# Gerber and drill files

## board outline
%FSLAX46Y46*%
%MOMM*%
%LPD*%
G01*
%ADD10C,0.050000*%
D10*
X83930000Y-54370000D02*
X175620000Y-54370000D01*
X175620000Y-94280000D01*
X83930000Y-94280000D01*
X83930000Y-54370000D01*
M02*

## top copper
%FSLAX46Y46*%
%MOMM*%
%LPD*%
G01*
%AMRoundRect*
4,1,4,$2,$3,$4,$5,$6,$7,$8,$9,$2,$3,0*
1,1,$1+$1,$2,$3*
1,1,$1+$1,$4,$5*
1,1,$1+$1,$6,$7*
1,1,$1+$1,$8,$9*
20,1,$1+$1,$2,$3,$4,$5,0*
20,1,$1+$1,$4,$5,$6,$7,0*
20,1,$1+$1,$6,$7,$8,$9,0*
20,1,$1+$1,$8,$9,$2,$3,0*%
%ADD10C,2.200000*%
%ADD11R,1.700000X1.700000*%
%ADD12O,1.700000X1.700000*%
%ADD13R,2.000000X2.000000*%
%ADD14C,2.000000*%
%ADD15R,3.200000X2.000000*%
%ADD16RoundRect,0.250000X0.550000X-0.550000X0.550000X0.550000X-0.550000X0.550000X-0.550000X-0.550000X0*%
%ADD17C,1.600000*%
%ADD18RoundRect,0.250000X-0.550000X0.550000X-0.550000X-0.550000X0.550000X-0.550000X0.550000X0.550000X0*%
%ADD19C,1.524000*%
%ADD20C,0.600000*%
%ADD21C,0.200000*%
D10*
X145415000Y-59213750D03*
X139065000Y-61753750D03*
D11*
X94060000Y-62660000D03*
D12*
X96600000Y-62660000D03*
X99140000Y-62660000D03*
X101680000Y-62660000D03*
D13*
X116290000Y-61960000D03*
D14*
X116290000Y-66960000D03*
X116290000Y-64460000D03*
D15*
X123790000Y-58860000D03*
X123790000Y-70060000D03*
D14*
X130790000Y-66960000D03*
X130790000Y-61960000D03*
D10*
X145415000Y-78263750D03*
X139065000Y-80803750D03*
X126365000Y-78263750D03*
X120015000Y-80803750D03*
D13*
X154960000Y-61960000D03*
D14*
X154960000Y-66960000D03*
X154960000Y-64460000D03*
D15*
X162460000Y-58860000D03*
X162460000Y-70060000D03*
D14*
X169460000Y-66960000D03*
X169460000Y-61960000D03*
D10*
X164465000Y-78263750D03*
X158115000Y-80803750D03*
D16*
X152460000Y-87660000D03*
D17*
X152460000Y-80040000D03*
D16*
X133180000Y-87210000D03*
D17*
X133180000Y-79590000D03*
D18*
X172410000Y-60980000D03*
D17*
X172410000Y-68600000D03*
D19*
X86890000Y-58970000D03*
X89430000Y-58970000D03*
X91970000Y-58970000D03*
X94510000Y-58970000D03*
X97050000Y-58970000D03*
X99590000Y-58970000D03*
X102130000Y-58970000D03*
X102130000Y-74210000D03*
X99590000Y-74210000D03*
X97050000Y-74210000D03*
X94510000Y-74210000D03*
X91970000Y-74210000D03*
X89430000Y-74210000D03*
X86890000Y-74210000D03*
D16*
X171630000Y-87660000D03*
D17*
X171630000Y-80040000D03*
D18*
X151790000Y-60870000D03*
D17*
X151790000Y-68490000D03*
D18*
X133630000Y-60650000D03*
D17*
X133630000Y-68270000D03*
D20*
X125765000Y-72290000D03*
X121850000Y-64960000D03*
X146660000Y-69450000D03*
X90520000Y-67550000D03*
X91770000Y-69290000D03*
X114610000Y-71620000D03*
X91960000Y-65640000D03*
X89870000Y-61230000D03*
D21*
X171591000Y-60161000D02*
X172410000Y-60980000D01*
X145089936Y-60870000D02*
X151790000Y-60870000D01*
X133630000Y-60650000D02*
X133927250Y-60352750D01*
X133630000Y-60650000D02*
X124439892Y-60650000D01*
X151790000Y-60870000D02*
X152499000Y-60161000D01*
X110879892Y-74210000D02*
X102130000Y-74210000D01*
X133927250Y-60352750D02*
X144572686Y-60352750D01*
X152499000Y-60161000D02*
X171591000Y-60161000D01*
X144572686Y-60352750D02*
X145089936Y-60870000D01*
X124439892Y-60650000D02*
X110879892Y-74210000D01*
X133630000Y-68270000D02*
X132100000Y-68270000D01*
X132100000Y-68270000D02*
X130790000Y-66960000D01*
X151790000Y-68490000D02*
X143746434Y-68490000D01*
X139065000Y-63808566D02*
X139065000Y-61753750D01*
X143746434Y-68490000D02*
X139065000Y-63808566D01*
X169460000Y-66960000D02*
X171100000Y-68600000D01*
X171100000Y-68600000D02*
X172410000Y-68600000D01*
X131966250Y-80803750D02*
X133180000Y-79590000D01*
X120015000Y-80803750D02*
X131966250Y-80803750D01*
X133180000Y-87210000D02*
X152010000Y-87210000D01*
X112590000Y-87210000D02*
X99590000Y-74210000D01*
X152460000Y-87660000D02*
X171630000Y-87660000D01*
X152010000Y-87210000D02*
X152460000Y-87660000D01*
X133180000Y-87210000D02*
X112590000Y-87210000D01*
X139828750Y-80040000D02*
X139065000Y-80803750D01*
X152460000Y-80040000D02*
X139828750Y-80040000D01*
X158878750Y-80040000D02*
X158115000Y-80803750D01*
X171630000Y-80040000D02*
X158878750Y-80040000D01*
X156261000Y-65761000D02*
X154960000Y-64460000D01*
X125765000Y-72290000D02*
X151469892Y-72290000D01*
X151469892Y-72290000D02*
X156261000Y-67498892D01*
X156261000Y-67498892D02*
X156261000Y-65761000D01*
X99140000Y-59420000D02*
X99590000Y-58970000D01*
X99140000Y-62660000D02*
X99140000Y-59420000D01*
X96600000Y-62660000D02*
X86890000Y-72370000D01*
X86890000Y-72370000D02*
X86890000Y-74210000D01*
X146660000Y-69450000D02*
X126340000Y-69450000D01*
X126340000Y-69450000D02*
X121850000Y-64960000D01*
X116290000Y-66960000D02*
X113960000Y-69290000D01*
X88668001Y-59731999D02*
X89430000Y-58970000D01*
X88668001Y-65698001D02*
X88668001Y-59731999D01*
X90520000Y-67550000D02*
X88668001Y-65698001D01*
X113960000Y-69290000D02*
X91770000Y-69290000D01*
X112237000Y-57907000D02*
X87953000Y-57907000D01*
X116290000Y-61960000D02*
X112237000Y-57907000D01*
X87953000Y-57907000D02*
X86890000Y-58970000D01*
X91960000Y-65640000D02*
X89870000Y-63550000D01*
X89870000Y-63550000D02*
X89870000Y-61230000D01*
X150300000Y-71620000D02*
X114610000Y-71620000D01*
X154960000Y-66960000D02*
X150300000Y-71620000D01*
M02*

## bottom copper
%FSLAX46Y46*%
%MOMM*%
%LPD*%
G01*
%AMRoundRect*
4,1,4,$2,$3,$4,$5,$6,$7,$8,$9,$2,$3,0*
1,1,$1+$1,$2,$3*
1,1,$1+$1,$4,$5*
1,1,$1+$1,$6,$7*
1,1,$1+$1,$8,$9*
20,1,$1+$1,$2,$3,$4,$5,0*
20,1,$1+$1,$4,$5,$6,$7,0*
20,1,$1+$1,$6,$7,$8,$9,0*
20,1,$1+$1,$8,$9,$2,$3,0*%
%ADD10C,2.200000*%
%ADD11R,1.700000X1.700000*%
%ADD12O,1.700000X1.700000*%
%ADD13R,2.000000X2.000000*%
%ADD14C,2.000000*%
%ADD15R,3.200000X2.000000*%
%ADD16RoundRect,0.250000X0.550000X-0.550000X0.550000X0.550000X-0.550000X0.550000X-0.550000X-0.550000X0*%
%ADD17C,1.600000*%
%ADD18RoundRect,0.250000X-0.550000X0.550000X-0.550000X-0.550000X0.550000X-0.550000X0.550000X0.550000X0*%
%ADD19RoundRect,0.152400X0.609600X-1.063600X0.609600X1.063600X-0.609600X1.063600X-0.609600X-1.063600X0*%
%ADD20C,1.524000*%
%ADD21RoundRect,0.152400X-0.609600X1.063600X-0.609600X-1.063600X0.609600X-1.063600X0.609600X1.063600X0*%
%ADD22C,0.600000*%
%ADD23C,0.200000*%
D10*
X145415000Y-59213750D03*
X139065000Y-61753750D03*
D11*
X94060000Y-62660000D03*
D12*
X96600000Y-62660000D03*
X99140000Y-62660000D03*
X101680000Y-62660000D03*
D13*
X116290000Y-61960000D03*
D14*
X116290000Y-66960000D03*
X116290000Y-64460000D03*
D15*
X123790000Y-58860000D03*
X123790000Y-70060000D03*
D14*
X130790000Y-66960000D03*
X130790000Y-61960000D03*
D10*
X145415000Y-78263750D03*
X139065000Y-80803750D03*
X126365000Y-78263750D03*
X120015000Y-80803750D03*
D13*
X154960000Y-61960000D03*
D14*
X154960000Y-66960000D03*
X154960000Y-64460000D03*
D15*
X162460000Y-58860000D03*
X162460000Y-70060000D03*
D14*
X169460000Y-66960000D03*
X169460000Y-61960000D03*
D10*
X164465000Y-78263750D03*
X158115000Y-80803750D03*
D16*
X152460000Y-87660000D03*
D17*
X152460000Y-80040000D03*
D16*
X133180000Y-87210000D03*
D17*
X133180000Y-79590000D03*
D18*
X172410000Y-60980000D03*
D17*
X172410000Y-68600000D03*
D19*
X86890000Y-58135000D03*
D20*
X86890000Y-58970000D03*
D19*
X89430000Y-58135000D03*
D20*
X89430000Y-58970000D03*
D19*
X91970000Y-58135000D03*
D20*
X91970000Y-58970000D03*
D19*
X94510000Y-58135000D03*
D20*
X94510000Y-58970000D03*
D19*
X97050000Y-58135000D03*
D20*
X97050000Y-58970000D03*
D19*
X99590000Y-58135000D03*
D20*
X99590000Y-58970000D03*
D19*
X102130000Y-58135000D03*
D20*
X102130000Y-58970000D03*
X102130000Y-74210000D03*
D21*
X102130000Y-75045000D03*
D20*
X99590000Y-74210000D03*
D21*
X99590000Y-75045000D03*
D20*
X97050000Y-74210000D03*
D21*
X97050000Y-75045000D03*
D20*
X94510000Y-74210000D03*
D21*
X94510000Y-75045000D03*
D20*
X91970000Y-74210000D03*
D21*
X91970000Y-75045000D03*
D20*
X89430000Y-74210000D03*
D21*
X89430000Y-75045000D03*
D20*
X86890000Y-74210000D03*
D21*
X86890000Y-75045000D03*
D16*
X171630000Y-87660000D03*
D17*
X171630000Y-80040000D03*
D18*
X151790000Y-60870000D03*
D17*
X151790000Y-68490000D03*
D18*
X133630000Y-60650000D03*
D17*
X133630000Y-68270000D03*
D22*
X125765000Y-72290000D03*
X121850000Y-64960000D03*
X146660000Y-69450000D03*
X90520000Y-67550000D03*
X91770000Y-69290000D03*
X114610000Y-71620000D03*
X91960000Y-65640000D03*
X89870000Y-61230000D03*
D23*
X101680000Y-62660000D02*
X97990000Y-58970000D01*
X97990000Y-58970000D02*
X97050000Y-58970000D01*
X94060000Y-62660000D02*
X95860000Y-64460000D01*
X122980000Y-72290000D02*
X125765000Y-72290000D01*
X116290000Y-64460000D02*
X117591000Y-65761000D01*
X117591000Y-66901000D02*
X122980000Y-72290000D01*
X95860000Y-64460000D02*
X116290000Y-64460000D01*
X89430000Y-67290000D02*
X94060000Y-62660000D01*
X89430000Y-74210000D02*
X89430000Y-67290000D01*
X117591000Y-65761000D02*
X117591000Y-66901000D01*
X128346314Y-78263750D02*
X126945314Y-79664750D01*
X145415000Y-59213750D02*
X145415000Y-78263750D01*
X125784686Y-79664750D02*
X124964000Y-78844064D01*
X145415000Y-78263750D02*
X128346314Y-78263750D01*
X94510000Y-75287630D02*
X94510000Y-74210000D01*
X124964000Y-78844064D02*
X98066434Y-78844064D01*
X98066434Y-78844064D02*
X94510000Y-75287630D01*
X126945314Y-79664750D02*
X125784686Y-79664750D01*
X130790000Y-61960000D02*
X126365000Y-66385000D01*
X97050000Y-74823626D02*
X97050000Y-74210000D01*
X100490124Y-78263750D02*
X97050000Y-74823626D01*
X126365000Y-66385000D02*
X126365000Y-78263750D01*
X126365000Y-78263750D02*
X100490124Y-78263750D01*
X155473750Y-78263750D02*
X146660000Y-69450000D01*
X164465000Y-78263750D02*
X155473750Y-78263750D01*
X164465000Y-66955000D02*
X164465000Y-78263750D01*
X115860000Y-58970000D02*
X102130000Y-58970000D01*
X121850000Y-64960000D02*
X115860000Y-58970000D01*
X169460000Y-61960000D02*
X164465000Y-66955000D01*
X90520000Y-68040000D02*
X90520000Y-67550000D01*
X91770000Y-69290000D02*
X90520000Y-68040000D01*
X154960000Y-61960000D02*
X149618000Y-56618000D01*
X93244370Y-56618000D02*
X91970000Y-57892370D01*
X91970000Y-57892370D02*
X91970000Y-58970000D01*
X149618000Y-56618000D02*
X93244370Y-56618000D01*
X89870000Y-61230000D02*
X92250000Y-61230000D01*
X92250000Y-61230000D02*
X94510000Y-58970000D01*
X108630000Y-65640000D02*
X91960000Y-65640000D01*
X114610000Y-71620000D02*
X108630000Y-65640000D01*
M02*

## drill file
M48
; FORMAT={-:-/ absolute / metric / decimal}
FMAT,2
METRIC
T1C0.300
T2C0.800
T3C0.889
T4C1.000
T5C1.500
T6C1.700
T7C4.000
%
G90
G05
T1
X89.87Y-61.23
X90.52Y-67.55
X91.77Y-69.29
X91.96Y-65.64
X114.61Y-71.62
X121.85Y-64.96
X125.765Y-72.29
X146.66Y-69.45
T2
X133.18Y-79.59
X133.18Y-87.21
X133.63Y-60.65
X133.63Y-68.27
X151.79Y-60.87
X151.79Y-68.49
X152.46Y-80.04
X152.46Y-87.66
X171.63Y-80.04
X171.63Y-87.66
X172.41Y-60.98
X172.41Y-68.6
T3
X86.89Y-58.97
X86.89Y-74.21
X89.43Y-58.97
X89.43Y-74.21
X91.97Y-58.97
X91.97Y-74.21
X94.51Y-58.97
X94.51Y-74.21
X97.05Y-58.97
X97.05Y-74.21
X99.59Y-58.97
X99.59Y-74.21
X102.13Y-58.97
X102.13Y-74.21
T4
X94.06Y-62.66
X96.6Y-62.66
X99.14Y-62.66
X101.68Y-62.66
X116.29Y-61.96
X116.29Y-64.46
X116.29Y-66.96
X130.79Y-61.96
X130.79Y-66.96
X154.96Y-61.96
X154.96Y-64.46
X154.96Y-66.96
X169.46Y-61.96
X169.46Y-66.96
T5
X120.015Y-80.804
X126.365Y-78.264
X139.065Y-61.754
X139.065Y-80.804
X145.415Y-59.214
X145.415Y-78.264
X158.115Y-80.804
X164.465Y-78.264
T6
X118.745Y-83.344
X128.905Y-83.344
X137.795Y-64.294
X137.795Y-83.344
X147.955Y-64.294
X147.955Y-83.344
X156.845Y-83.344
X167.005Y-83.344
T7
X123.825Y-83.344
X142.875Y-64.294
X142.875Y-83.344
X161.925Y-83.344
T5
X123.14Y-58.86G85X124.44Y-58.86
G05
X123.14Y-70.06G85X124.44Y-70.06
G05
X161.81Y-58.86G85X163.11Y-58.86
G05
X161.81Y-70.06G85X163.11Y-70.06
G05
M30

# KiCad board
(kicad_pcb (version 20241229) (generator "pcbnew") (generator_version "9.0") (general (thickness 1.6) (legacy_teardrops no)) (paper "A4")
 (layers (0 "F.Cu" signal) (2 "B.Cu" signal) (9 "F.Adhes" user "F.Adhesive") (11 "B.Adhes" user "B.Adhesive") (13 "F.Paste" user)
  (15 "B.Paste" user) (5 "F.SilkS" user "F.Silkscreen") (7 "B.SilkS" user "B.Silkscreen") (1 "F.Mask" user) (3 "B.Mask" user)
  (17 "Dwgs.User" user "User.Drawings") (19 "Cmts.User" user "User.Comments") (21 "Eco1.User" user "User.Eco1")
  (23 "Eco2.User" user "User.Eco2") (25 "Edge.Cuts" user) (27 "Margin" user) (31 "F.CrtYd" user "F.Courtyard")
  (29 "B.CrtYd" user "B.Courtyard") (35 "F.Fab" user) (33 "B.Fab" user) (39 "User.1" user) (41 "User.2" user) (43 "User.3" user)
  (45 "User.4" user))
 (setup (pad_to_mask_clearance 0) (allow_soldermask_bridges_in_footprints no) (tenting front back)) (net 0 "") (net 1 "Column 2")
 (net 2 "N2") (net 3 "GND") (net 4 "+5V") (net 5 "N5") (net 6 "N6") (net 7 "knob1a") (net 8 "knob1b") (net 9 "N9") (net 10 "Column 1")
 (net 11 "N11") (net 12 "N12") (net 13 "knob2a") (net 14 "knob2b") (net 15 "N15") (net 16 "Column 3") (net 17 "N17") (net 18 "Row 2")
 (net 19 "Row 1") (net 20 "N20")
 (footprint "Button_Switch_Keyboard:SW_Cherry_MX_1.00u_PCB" (layer "F.Cu") (at 145.415 59.21375)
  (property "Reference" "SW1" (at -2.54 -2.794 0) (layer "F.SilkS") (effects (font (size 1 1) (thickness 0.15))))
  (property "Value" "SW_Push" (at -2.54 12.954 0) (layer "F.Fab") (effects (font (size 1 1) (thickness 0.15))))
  (pad "" np_thru_hole circle (at -7.62 5.08) (size 1.7 1.7) (drill 1.7) (layers "*.Cu" "*.Mask"))
  (pad "" np_thru_hole circle (at -2.54 5.08) (size 4 4) (drill 4) (layers "*.Cu" "*.Mask"))
  (pad "" np_thru_hole circle (at 2.54 5.08) (size 1.7 1.7) (drill 1.7) (layers "*.Cu" "*.Mask"))
  (pad "1" thru_hole circle (at 0 0) (size 2.2 2.2) (drill 1.5) (layers "*.Cu" "*.Mask") (remove_unused_layers no) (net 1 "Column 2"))
  (pad "2" thru_hole circle (at -6.35 2.54) (size 2.2 2.2) (drill 1.5) (layers "*.Cu" "*.Mask") (remove_unused_layers no) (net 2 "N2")))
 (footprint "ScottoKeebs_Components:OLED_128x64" (layer "F.Cu") (at 97.87 62.66)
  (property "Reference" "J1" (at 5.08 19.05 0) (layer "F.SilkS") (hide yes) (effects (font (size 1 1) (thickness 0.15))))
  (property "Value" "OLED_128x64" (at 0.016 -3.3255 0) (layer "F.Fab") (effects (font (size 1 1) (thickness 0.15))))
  (pad "1" thru_hole rect (at -3.81 0 90) (size 1.7 1.7) (drill 1) (layers "*.Cu" "*.Mask") (remove_unused_layers no) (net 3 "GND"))
  (pad "2" thru_hole oval (at -1.27 0 90) (size 1.7 1.7) (drill 1) (layers "*.Cu" "*.Mask") (remove_unused_layers no) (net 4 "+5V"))
  (pad "3" thru_hole oval (at 1.27 0 90) (size 1.7 1.7) (drill 1) (layers "*.Cu" "*.Mask") (remove_unused_layers no) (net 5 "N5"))
  (pad "4" thru_hole oval (at 3.81 0 90) (size 1.7 1.7) (drill 1) (layers "*.Cu" "*.Mask") (remove_unused_layers no) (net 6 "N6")))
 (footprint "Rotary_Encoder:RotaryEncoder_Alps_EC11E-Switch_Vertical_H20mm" (layer "F.Cu") (at 116.29 61.96)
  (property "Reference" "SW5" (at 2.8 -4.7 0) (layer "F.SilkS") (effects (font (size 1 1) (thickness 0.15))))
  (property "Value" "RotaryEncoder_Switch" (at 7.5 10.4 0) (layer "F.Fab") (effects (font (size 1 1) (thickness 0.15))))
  (pad "A" thru_hole rect (at 0 0) (size 2 2) (drill 1) (layers "*.Cu" "*.Mask") (remove_unused_layers no) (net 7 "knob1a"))
  (pad "B" thru_hole circle (at 0 5) (size 2 2) (drill 1) (layers "*.Cu" "*.Mask") (remove_unused_layers no) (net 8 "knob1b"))
  (pad "C" thru_hole circle (at 0 2.5) (size 2 2) (drill 1) (layers "*.Cu" "*.Mask") (remove_unused_layers no) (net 3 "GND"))
  (pad "MP" thru_hole rect (at 7.5 -3.1) (size 3.2 2) (drill oval 2.8 1.5) (layers "*.Cu" "*.Mask") (remove_unused_layers no))
  (pad "MP" thru_hole rect (at 7.5 8.1) (size 3.2 2) (drill oval 2.8 1.5) (layers "*.Cu" "*.Mask") (remove_unused_layers no))
  (pad "S1" thru_hole circle (at 14.5 5) (size 2 2) (drill 1) (layers "*.Cu" "*.Mask") (remove_unused_layers no) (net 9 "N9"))
  (pad "S2" thru_hole circle (at 14.5 0) (size 2 2) (drill 1) (layers "*.Cu" "*.Mask") (remove_unused_layers no) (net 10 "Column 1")))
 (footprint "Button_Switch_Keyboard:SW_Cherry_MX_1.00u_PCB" (layer "F.Cu") (at 145.415 78.26375)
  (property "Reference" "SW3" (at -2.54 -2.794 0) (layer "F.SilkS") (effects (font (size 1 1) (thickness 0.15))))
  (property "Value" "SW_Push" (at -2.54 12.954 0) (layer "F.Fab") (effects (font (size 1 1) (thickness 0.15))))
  (pad "" np_thru_hole circle (at -7.62 5.08) (size 1.7 1.7) (drill 1.7) (layers "*.Cu" "*.Mask"))
  (pad "" np_thru_hole circle (at -2.54 5.08) (size 4 4) (drill 4) (layers "*.Cu" "*.Mask"))
  (pad "" np_thru_hole circle (at 2.54 5.08) (size 1.7 1.7) (drill 1.7) (layers "*.Cu" "*.Mask"))
  (pad "1" thru_hole circle (at 0 0) (size 2.2 2.2) (drill 1.5) (layers "*.Cu" "*.Mask") (remove_unused_layers no) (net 1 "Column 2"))
  (pad "2" thru_hole circle (at -6.35 2.54) (size 2.2 2.2) (drill 1.5) (layers "*.Cu" "*.Mask") (remove_unused_layers no) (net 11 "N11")))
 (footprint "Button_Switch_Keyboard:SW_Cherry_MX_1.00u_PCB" (layer "F.Cu") (at 126.365 78.26375)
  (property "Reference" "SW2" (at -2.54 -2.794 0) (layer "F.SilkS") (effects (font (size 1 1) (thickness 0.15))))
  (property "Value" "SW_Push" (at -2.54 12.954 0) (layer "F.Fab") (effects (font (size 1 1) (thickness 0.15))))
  (pad "" np_thru_hole circle (at -7.62 5.08) (size 1.7 1.7) (drill 1.7) (layers "*.Cu" "*.Mask"))
  (pad "" np_thru_hole circle (at -2.54 5.08) (size 4 4) (drill 4) (layers "*.Cu" "*.Mask"))
  (pad "" np_thru_hole circle (at 2.54 5.08) (size 1.7 1.7) (drill 1.7) (layers "*.Cu" "*.Mask"))
  (pad "1" thru_hole circle (at 0 0) (size 2.2 2.2) (drill 1.5) (layers "*.Cu" "*.Mask") (remove_unused_layers no) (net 10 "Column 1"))
  (pad "2" thru_hole circle (at -6.35 2.54) (size 2.2 2.2) (drill 1.5) (layers "*.Cu" "*.Mask") (remove_unused_layers no) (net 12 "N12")))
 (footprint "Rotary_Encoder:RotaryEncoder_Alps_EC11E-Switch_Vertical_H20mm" (layer "F.Cu") (at 154.96 61.96)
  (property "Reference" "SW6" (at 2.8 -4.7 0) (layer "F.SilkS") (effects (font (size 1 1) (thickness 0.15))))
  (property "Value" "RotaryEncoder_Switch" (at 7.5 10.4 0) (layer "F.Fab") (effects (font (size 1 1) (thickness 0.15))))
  (pad "A" thru_hole rect (at 0 0) (size 2 2) (drill 1) (layers "*.Cu" "*.Mask") (remove_unused_layers no) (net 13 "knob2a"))
  (pad "B" thru_hole circle (at 0 5) (size 2 2) (drill 1) (layers "*.Cu" "*.Mask") (remove_unused_layers no) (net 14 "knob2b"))
  (pad "C" thru_hole circle (at 0 2.5) (size 2 2) (drill 1) (layers "*.Cu" "*.Mask") (remove_unused_layers no) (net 3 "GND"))
  (pad "MP" thru_hole rect (at 7.5 -3.1) (size 3.2 2) (drill oval 2.8 1.5) (layers "*.Cu" "*.Mask") (remove_unused_layers no))
  (pad "MP" thru_hole rect (at 7.5 8.1) (size 3.2 2) (drill oval 2.8 1.5) (layers "*.Cu" "*.Mask") (remove_unused_layers no))
  (pad "S1" thru_hole circle (at 14.5 5) (size 2 2) (drill 1) (layers "*.Cu" "*.Mask") (remove_unused_layers no) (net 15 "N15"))
  (pad "S2" thru_hole circle (at 14.5 0) (size 2 2) (drill 1) (layers "*.Cu" "*.Mask") (remove_unused_layers no) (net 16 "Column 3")))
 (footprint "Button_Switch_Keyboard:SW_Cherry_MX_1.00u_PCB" (layer "F.Cu") (at 164.465 78.26375)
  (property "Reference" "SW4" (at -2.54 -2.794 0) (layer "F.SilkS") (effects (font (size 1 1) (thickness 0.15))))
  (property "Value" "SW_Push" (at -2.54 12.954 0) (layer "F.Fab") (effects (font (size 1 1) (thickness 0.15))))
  (pad "" np_thru_hole circle (at -7.62 5.08) (size 1.7 1.7) (drill 1.7) (layers "*.Cu" "*.Mask"))
  (pad "" np_thru_hole circle (at -2.54 5.08) (size 4 4) (drill 4) (layers "*.Cu" "*.Mask"))
  (pad "" np_thru_hole circle (at 2.54 5.08) (size 1.7 1.7) (drill 1.7) (layers "*.Cu" "*.Mask"))
  (pad "1" thru_hole circle (at 0 0) (size 2.2 2.2) (drill 1.5) (layers "*.Cu" "*.Mask") (remove_unused_layers no) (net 16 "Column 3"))
  (pad "2" thru_hole circle (at -6.35 2.54) (size 2.2 2.2) (drill 1.5) (layers "*.Cu" "*.Mask") (remove_unused_layers no) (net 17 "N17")))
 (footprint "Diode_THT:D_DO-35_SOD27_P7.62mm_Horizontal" (layer "B.Cu") (at 152.46 87.66 90)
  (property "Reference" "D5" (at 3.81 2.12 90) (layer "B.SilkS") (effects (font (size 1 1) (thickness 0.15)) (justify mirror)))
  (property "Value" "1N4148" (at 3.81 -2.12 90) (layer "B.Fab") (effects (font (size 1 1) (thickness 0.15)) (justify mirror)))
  (pad "1" thru_hole roundrect (at 0 0 90) (size 1.6 1.6) (drill 0.8) (layers "*.Cu" "*.Mask") (remove_unused_layers no)
   (roundrect_rratio 0.15625) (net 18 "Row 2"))
  (pad "2" thru_hole circle (at 7.62 0 90) (size 1.6 1.6) (drill 0.8) (layers "*.Cu" "*.Mask") (remove_unused_layers no) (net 11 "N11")))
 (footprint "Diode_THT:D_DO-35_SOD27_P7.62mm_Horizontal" (layer "B.Cu") (at 133.18 87.21 90)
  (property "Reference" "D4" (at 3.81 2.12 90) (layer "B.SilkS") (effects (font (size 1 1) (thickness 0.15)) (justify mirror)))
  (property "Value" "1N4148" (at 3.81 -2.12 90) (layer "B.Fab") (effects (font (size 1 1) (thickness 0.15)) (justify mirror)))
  (pad "1" thru_hole roundrect (at 0 0 90) (size 1.6 1.6) (drill 0.8) (layers "*.Cu" "*.Mask") (remove_unused_layers no)
   (roundrect_rratio 0.15625) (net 18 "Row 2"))
  (pad "2" thru_hole circle (at 7.62 0 90) (size 1.6 1.6) (drill 0.8) (layers "*.Cu" "*.Mask") (remove_unused_layers no) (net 12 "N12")))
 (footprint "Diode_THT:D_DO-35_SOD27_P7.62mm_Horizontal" (layer "B.Cu") (at 172.41 60.98 -90)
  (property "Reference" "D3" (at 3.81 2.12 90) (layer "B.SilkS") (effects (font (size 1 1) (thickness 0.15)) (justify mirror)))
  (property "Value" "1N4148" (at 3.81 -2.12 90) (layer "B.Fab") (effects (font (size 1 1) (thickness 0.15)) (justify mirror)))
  (pad "1" thru_hole roundrect (at 0 0 270) (size 1.6 1.6) (drill 0.8) (layers "*.Cu" "*.Mask") (remove_unused_layers no)
   (roundrect_rratio 0.15625) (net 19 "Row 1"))
  (pad "2" thru_hole circle (at 7.62 0 270) (size 1.6 1.6) (drill 0.8) (layers "*.Cu" "*.Mask") (remove_unused_layers no) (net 15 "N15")))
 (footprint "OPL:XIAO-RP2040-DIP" (layer "B.Cu") (at 94.51 66.59 -90)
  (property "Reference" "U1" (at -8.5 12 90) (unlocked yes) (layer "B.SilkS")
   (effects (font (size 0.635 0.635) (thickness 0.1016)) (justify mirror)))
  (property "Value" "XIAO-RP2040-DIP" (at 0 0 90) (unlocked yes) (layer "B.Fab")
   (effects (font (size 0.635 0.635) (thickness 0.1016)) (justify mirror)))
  (pad "1" smd roundrect (at -8.455 7.62 90) (size 2.432 1.524) (layers "B.Cu" "B.Mask") (roundrect_rratio 0.1) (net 7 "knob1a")
   (thermal_bridge_angle 45))
  (pad "1" thru_hole circle (at -7.62 7.62 90) (size 1.524 1.524) (drill 0.889) (layers "*.Cu" "*.Mask") (remove_unused_layers no)
   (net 7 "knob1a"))
  (pad "2" smd roundrect (at -8.455 5.08 90) (size 2.432 1.524) (layers "B.Cu" "B.Mask") (roundrect_rratio 0.1) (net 8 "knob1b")
   (thermal_bridge_angle 45))
  (pad "2" thru_hole circle (at -7.62 5.08 90) (size 1.524 1.524) (drill 0.889) (layers "*.Cu" "*.Mask") (remove_unused_layers no)
   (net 8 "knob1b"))
  (pad "3" smd roundrect (at -8.455 2.54 90) (size 2.432 1.524) (layers "B.Cu" "B.Mask") (roundrect_rratio 0.1) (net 13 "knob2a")
   (thermal_bridge_angle 45))
  (pad "3" thru_hole circle (at -7.62 2.54 90) (size 1.524 1.524) (drill 0.889) (layers "*.Cu" "*.Mask") (remove_unused_layers no)
   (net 13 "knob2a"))
  (pad "4" smd roundrect (at -8.455 0 90) (size 2.432 1.524) (layers "B.Cu" "B.Mask") (roundrect_rratio 0.1) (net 14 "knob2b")
   (thermal_bridge_angle 45))
  (pad "4" thru_hole circle (at -7.62 0 90) (size 1.524 1.524) (drill 0.889) (layers "*.Cu" "*.Mask") (remove_unused_layers no)
   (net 14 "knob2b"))
  (pad "5" smd roundrect (at -8.455 -2.54 90) (size 2.432 1.524) (layers "B.Cu" "B.Mask") (roundrect_rratio 0.1) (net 6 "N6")
   (thermal_bridge_angle 45))
  (pad "5" thru_hole circle (at -7.62 -2.54 90) (size 1.524 1.524) (drill 0.889) (layers "*.Cu" "*.Mask") (remove_unused_layers no)
   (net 6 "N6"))
  (pad "6" smd roundrect (at -8.455 -5.08 90) (size 2.432 1.524) (layers "B.Cu" "B.Mask") (roundrect_rratio 0.1) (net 5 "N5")
   (thermal_bridge_angle 45))
  (pad "6" thru_hole circle (at -7.62 -5.08 90) (size 1.524 1.524) (drill 0.889) (layers "*.Cu" "*.Mask") (remove_unused_layers no)
   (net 5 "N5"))
  (pad "7" smd roundrect (at -8.455 -7.62 90) (size 2.432 1.524) (layers "B.Cu" "B.Mask") (roundrect_rratio 0.1) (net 16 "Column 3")
   (thermal_bridge_angle 45))
  (pad "7" thru_hole circle (at -7.62 -7.62 90) (size 1.524 1.524) (drill 0.889) (layers "*.Cu" "*.Mask") (remove_unused_layers no)
   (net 16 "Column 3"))
  (pad "8" thru_hole circle (at 7.62 -7.62 270) (size 1.524 1.524) (drill 0.889) (layers "*.Cu" "*.Mask") (remove_unused_layers no)
   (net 19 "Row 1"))
  (pad "8" smd roundrect (at 8.455 -7.62 270) (size 2.432 1.524) (layers "B.Cu" "B.Mask") (roundrect_rratio 0.1) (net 19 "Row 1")
   (thermal_bridge_angle 45))
  (pad "9" thru_hole circle (at 7.62 -5.08 270) (size 1.524 1.524) (drill 0.889) (layers "*.Cu" "*.Mask") (remove_unused_layers no)
   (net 18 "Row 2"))
  (pad "9" smd roundrect (at 8.455 -5.08 270) (size 2.432 1.524) (layers "B.Cu" "B.Mask") (roundrect_rratio 0.1) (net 18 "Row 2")
   (thermal_bridge_angle 45))
  (pad "10" thru_hole circle (at 7.62 -2.54 270) (size 1.524 1.524) (drill 0.889) (layers "*.Cu" "*.Mask") (remove_unused_layers no)
   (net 10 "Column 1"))
  (pad "10" smd roundrect (at 8.455 -2.54 270) (size 2.432 1.524) (layers "B.Cu" "B.Mask") (roundrect_rratio 0.1) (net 10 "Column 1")
   (thermal_bridge_angle 45))
  (pad "11" thru_hole circle (at 7.62 0 270) (size 1.524 1.524) (drill 0.889) (layers "*.Cu" "*.Mask") (remove_unused_layers no)
   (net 1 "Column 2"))
  (pad "11" smd roundrect (at 8.455 0 270) (size 2.432 1.524) (layers "B.Cu" "B.Mask") (roundrect_rratio 0.1) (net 1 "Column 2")
   (thermal_bridge_angle 45))
  (pad "12" thru_hole circle (at 7.62 2.54 270) (size 1.524 1.524) (drill 0.889) (layers "*.Cu" "*.Mask") (remove_unused_layers no)
   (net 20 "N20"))
  (pad "12" smd roundrect (at 8.455 2.54 270) (size 2.432 1.524) (layers "B.Cu" "B.Mask") (roundrect_rratio 0.1) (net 20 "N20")
   (thermal_bridge_angle 45))
  (pad "13" thru_hole circle (at 7.62 5.08 270) (size 1.524 1.524) (drill 0.889) (layers "*.Cu" "*.Mask") (remove_unused_layers no)
   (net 3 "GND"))
  (pad "13" smd roundrect (at 8.455 5.08 270) (size 2.432 1.524) (layers "B.Cu" "B.Mask") (roundrect_rratio 0.1) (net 3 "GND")
   (thermal_bridge_angle 45))
  (pad "14" thru_hole circle (at 7.62 7.62 270) (size 1.524 1.524) (drill 0.889) (layers "*.Cu" "*.Mask") (remove_unused_layers no)
   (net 4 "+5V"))
  (pad "14" smd roundrect (at 8.455 7.62 270) (size 2.432 1.524) (layers "B.Cu" "B.Mask") (roundrect_rratio 0.1) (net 4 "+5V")
   (thermal_bridge_angle 45)))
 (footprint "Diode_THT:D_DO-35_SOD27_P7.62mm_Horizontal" (layer "B.Cu") (at 171.63 87.66 90)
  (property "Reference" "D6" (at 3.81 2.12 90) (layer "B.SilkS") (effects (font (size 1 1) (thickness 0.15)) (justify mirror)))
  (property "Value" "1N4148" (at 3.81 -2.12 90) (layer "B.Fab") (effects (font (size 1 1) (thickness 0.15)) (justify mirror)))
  (pad "1" thru_hole roundrect (at 0 0 90) (size 1.6 1.6) (drill 0.8) (layers "*.Cu" "*.Mask") (remove_unused_layers no)
   (roundrect_rratio 0.15625) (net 18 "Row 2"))
  (pad "2" thru_hole circle (at 7.62 0 90) (size 1.6 1.6) (drill 0.8) (layers "*.Cu" "*.Mask") (remove_unused_layers no) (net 17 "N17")))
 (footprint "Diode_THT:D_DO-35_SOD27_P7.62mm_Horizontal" (layer "B.Cu") (at 151.79 60.87 -90)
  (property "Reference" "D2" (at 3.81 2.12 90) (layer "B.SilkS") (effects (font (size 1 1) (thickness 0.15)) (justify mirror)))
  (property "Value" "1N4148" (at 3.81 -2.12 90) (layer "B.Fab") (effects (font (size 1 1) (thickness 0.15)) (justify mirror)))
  (pad "1" thru_hole roundrect (at 0 0 270) (size 1.6 1.6) (drill 0.8) (layers "*.Cu" "*.Mask") (remove_unused_layers no)
   (roundrect_rratio 0.15625) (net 19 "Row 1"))
  (pad "2" thru_hole circle (at 7.62 0 270) (size 1.6 1.6) (drill 0.8) (layers "*.Cu" "*.Mask") (remove_unused_layers no) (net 2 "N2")))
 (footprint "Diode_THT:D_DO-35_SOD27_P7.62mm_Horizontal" (layer "B.Cu") (at 133.63 60.65 -90)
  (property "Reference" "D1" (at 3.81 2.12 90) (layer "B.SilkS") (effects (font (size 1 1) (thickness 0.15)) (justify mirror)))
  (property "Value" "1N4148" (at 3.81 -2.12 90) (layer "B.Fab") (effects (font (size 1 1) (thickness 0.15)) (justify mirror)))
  (pad "1" thru_hole roundrect (at 0 0 270) (size 1.6 1.6) (drill 0.8) (layers "*.Cu" "*.Mask") (remove_unused_layers no)
   (roundrect_rratio 0.15625) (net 19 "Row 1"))
  (pad "2" thru_hole circle (at 7.62 0 270) (size 1.6 1.6) (drill 0.8) (layers "*.Cu" "*.Mask") (remove_unused_layers no) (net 9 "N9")))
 (gr_rect (start 83.93 54.37) (end 175.62 94.28) (stroke (width 0.05) (type default)) (fill no) (layer "Edge.Cuts"))
 (segment (start 171.591 60.161) (end 172.41 60.98) (width 0.2) (layer "F.Cu") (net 19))
 (segment (start 145.089936 60.87) (end 151.79 60.87) (width 0.2) (layer "F.Cu") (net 19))
 (segment (start 133.63 60.65) (end 133.92725 60.35275) (width 0.2) (layer "F.Cu") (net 19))
 (segment (start 133.63 60.65) (end 124.439892 60.65) (width 0.2) (layer "F.Cu") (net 19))
 (segment (start 151.79 60.87) (end 152.499 60.161) (width 0.2) (layer "F.Cu") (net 19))
 (segment (start 110.879892 74.21) (end 102.13 74.21) (width 0.2) (layer "F.Cu") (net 19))
 (segment (start 133.92725 60.35275) (end 144.572686 60.35275) (width 0.2) (layer "F.Cu") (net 19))
 (segment (start 152.499 60.161) (end 171.591 60.161) (width 0.2) (layer "F.Cu") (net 19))
 (segment (start 144.572686 60.35275) (end 145.089936 60.87) (width 0.2) (layer "F.Cu") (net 19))
 (segment (start 124.439892 60.65) (end 110.879892 74.21) (width 0.2) (layer "F.Cu") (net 19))
 (segment (start 133.63 68.27) (end 132.1 68.27) (width 0.2) (layer "F.Cu") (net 9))
 (segment (start 132.1 68.27) (end 130.79 66.96) (width 0.2) (layer "F.Cu") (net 9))
 (segment (start 151.79 68.49) (end 143.746434 68.49) (width 0.2) (layer "F.Cu") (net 2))
 (segment (start 139.065 63.808566) (end 139.065 61.75375) (width 0.2) (layer "F.Cu") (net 2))
 (segment (start 143.746434 68.49) (end 139.065 63.808566) (width 0.2) (layer "F.Cu") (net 2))
 (segment (start 169.46 66.96) (end 171.1 68.6) (width 0.2) (layer "F.Cu") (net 15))
 (segment (start 171.1 68.6) (end 172.41 68.6) (width 0.2) (layer "F.Cu") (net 15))
 (segment (start 131.96625 80.80375) (end 133.18 79.59) (width 0.2) (layer "F.Cu") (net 12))
 (segment (start 120.015 80.80375) (end 131.96625 80.80375) (width 0.2) (layer "F.Cu") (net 12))
 (segment (start 133.18 87.21) (end 152.01 87.21) (width 0.2) (layer "F.Cu") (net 18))
 (segment (start 112.59 87.21) (end 99.59 74.21) (width 0.2) (layer "F.Cu") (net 18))
 (segment (start 152.46 87.66) (end 171.63 87.66) (width 0.2) (layer "F.Cu") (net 18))
 (segment (start 152.01 87.21) (end 152.46 87.66) (width 0.2) (layer "F.Cu") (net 18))
 (segment (start 133.18 87.21) (end 112.59 87.21) (width 0.2) (layer "F.Cu") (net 18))
 (segment (start 139.82875 80.04) (end 139.065 80.80375) (width 0.2) (layer "F.Cu") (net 11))
 (segment (start 152.46 80.04) (end 139.82875 80.04) (width 0.2) (layer "F.Cu") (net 11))
 (segment (start 158.87875 80.04) (end 158.115 80.80375) (width 0.2) (layer "F.Cu") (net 17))
 (segment (start 171.63 80.04) (end 158.87875 80.04) (width 0.2) (layer "F.Cu") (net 17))
 (segment (start 101.68 62.66) (end 97.99 58.97) (width 0.2) (layer "B.Cu") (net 6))
 (segment (start 97.99 58.97) (end 97.05 58.97) (width 0.2) (layer "B.Cu") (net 6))
 (segment (start 156.261 65.761) (end 154.96 64.46) (width 0.2) (layer "F.Cu") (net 3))
 (segment (start 125.765 72.29) (end 151.469892 72.29) (width 0.2) (layer "F.Cu") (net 3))
 (segment (start 151.469892 72.29) (end 156.261 67.498892) (width 0.2) (layer "F.Cu") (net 3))
 (segment (start 156.261 67.498892) (end 156.261 65.761) (width 0.2) (layer "F.Cu") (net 3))
 (via (at 125.765 72.29) (size 0.6) (drill 0.3) (layers "F.Cu" "B.Cu") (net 3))
 (segment (start 94.06 62.66) (end 95.86 64.46) (width 0.2) (layer "B.Cu") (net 3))
 (segment (start 122.98 72.29) (end 125.765 72.29) (width 0.2) (layer "B.Cu") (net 3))
 (segment (start 116.29 64.46) (end 117.591 65.761) (width 0.2) (layer "B.Cu") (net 3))
 (segment (start 117.591 66.901) (end 122.98 72.29) (width 0.2) (layer "B.Cu") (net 3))
 (segment (start 95.86 64.46) (end 116.29 64.46) (width 0.2) (layer "B.Cu") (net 3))
 (segment (start 89.43 67.29) (end 94.06 62.66) (width 0.2) (layer "B.Cu") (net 3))
 (segment (start 89.43 74.21) (end 89.43 67.29) (width 0.2) (layer "B.Cu") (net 3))
 (segment (start 117.591 65.761) (end 117.591 66.901) (width 0.2) (layer "B.Cu") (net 3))
 (segment (start 99.14 59.42) (end 99.59 58.97) (width 0.2) (layer "F.Cu") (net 5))
 (segment (start 99.14 62.66) (end 99.14 59.42) (width 0.2) (layer "F.Cu") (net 5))
 (segment (start 96.6 62.66) (end 86.89 72.37) (width 0.2) (layer "F.Cu") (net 4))
 (segment (start 86.89 72.37) (end 86.89 74.21) (width 0.2) (layer "F.Cu") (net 4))
 (segment (start 128.346314 78.26375) (end 126.945314 79.66475) (width 0.2) (layer "B.Cu") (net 1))
 (segment (start 145.415 59.21375) (end 145.415 78.26375) (width 0.2) (layer "B.Cu") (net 1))
 (segment (start 125.784686 79.66475) (end 124.964 78.844064) (width 0.2) (layer "B.Cu") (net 1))
 (segment (start 145.415 78.26375) (end 128.346314 78.26375) (width 0.2) (layer "B.Cu") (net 1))
 (segment (start 94.51 75.28763) (end 94.51 74.21) (width 0.2) (layer "B.Cu") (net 1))
 (segment (start 124.964 78.844064) (end 98.066434 78.844064) (width 0.2) (layer "B.Cu") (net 1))
 (segment (start 98.066434 78.844064) (end 94.51 75.28763) (width 0.2) (layer "B.Cu") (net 1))
 (segment (start 126.945314 79.66475) (end 125.784686 79.66475) (width 0.2) (layer "B.Cu") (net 1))
 (segment (start 130.79 61.96) (end 126.365 66.385) (width 0.2) (layer "B.Cu") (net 10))
 (segment (start 97.05 74.823626) (end 97.05 74.21) (width 0.2) (layer "B.Cu") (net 10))
 (segment (start 100.490124 78.26375) (end 97.05 74.823626) (width 0.2) (layer "B.Cu") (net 10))
 (segment (start 126.365 66.385) (end 126.365 78.26375) (width 0.2) (layer "B.Cu") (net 10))
 (segment (start 126.365 78.26375) (end 100.490124 78.26375) (width 0.2) (layer "B.Cu") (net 10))
 (segment (start 146.66 69.45) (end 126.34 69.45) (width 0.2) (layer "F.Cu") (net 16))
 (segment (start 126.34 69.45) (end 121.85 64.96) (width 0.2) (layer "F.Cu") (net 16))
 (via (at 121.85 64.96) (size 0.6) (drill 0.3) (layers "F.Cu" "B.Cu") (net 16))
 (via (at 146.66 69.45) (size 0.6) (drill 0.3) (layers "F.Cu" "B.Cu") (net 16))
 (segment (start 155.47375 78.26375) (end 146.66 69.45) (width 0.2) (layer "B.Cu") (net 16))
 (segment (start 164.465 78.26375) (end 155.47375 78.26375) (width 0.2) (layer "B.Cu") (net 16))
 (segment (start 164.465 66.955) (end 164.465 78.26375) (width 0.2) (layer "B.Cu") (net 16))
 (segment (start 115.86 58.97) (end 102.13 58.97) (width 0.2) (layer "B.Cu") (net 16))
 (segment (start 121.85 64.96) (end 115.86 58.97) (width 0.2) (layer "B.Cu") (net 16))
 (segment (start 169.46 61.96) (end 164.465 66.955) (width 0.2) (layer "B.Cu") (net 16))
 (segment (start 116.29 66.96) (end 113.96 69.29) (width 0.2) (layer "F.Cu") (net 8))
 (segment (start 88.668001 59.731999) (end 89.43 58.97) (width 0.2) (layer "F.Cu") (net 8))
 (segment (start 88.668001 65.698001) (end 88.668001 59.731999) (width 0.2) (layer "F.Cu") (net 8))
 (segment (start 90.52 67.55) (end 88.668001 65.698001) (width 0.2) (layer "F.Cu") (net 8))
 (segment (start 113.96 69.29) (end 91.77 69.29) (width 0.2) (layer "F.Cu") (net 8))
 (via (at 90.52 67.55) (size 0.6) (drill 0.3) (layers "F.Cu" "B.Cu") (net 8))
 (via (at 91.77 69.29) (size 0.6) (drill 0.3) (layers "F.Cu" "B.Cu") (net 8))
 (segment (start 90.52 68.04) (end 90.52 67.55) (width 0.2) (layer "B.Cu") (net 8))
 (segment (start 91.77 69.29) (end 90.52 68.04) (width 0.2) (layer "B.Cu") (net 8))
 (segment (start 112.237 57.907) (end 87.953 57.907) (width 0.2) (layer "F.Cu") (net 7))
 (segment (start 116.29 61.96) (end 112.237 57.907) (width 0.2) (layer "F.Cu") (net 7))
 (segment (start 87.953 57.907) (end 86.89 58.97) (width 0.2) (layer "F.Cu") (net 7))
 (segment (start 154.96 61.96) (end 149.618 56.618) (width 0.2) (layer "B.Cu") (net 13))
 (segment (start 93.24437 56.618) (end 91.97 57.89237) (width 0.2) (layer "B.Cu") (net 13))
 (segment (start 91.97 57.89237) (end 91.97 58.97) (width 0.2) (layer "B.Cu") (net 13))
 (segment (start 149.618 56.618) (end 93.24437 56.618) (width 0.2) (layer "B.Cu") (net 13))
 (segment (start 91.96 65.64) (end 89.87 63.55) (width 0.2) (layer "F.Cu") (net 14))
 (segment (start 89.87 63.55) (end 89.87 61.23) (width 0.2) (layer "F.Cu") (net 14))
 (segment (start 150.3 71.62) (end 114.61 71.62) (width 0.2) (layer "F.Cu") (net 14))
 (segment (start 154.96 66.96) (end 150.3 71.62) (width 0.2) (layer "F.Cu") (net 14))
 (via (at 114.61 71.62) (size 0.6) (drill 0.3) (layers "F.Cu" "B.Cu") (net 14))
 (via (at 91.96 65.64) (size 0.6) (drill 0.3) (layers "F.Cu" "B.Cu") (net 14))
 (via (at 89.87 61.23) (size 0.6) (drill 0.3) (layers "F.Cu" "B.Cu") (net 14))
 (segment (start 89.87 61.23) (end 92.25 61.23) (width 0.2) (layer "B.Cu") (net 14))
 (segment (start 92.25 61.23) (end 94.51 58.97) (width 0.2) (layer "B.Cu") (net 14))
 (segment (start 108.63 65.64) (end 91.96 65.64) (width 0.2) (layer "B.Cu") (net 14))
 (segment (start 114.61 71.62) (end 108.63 65.64) (width 0.2) (layer "B.Cu") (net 14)))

